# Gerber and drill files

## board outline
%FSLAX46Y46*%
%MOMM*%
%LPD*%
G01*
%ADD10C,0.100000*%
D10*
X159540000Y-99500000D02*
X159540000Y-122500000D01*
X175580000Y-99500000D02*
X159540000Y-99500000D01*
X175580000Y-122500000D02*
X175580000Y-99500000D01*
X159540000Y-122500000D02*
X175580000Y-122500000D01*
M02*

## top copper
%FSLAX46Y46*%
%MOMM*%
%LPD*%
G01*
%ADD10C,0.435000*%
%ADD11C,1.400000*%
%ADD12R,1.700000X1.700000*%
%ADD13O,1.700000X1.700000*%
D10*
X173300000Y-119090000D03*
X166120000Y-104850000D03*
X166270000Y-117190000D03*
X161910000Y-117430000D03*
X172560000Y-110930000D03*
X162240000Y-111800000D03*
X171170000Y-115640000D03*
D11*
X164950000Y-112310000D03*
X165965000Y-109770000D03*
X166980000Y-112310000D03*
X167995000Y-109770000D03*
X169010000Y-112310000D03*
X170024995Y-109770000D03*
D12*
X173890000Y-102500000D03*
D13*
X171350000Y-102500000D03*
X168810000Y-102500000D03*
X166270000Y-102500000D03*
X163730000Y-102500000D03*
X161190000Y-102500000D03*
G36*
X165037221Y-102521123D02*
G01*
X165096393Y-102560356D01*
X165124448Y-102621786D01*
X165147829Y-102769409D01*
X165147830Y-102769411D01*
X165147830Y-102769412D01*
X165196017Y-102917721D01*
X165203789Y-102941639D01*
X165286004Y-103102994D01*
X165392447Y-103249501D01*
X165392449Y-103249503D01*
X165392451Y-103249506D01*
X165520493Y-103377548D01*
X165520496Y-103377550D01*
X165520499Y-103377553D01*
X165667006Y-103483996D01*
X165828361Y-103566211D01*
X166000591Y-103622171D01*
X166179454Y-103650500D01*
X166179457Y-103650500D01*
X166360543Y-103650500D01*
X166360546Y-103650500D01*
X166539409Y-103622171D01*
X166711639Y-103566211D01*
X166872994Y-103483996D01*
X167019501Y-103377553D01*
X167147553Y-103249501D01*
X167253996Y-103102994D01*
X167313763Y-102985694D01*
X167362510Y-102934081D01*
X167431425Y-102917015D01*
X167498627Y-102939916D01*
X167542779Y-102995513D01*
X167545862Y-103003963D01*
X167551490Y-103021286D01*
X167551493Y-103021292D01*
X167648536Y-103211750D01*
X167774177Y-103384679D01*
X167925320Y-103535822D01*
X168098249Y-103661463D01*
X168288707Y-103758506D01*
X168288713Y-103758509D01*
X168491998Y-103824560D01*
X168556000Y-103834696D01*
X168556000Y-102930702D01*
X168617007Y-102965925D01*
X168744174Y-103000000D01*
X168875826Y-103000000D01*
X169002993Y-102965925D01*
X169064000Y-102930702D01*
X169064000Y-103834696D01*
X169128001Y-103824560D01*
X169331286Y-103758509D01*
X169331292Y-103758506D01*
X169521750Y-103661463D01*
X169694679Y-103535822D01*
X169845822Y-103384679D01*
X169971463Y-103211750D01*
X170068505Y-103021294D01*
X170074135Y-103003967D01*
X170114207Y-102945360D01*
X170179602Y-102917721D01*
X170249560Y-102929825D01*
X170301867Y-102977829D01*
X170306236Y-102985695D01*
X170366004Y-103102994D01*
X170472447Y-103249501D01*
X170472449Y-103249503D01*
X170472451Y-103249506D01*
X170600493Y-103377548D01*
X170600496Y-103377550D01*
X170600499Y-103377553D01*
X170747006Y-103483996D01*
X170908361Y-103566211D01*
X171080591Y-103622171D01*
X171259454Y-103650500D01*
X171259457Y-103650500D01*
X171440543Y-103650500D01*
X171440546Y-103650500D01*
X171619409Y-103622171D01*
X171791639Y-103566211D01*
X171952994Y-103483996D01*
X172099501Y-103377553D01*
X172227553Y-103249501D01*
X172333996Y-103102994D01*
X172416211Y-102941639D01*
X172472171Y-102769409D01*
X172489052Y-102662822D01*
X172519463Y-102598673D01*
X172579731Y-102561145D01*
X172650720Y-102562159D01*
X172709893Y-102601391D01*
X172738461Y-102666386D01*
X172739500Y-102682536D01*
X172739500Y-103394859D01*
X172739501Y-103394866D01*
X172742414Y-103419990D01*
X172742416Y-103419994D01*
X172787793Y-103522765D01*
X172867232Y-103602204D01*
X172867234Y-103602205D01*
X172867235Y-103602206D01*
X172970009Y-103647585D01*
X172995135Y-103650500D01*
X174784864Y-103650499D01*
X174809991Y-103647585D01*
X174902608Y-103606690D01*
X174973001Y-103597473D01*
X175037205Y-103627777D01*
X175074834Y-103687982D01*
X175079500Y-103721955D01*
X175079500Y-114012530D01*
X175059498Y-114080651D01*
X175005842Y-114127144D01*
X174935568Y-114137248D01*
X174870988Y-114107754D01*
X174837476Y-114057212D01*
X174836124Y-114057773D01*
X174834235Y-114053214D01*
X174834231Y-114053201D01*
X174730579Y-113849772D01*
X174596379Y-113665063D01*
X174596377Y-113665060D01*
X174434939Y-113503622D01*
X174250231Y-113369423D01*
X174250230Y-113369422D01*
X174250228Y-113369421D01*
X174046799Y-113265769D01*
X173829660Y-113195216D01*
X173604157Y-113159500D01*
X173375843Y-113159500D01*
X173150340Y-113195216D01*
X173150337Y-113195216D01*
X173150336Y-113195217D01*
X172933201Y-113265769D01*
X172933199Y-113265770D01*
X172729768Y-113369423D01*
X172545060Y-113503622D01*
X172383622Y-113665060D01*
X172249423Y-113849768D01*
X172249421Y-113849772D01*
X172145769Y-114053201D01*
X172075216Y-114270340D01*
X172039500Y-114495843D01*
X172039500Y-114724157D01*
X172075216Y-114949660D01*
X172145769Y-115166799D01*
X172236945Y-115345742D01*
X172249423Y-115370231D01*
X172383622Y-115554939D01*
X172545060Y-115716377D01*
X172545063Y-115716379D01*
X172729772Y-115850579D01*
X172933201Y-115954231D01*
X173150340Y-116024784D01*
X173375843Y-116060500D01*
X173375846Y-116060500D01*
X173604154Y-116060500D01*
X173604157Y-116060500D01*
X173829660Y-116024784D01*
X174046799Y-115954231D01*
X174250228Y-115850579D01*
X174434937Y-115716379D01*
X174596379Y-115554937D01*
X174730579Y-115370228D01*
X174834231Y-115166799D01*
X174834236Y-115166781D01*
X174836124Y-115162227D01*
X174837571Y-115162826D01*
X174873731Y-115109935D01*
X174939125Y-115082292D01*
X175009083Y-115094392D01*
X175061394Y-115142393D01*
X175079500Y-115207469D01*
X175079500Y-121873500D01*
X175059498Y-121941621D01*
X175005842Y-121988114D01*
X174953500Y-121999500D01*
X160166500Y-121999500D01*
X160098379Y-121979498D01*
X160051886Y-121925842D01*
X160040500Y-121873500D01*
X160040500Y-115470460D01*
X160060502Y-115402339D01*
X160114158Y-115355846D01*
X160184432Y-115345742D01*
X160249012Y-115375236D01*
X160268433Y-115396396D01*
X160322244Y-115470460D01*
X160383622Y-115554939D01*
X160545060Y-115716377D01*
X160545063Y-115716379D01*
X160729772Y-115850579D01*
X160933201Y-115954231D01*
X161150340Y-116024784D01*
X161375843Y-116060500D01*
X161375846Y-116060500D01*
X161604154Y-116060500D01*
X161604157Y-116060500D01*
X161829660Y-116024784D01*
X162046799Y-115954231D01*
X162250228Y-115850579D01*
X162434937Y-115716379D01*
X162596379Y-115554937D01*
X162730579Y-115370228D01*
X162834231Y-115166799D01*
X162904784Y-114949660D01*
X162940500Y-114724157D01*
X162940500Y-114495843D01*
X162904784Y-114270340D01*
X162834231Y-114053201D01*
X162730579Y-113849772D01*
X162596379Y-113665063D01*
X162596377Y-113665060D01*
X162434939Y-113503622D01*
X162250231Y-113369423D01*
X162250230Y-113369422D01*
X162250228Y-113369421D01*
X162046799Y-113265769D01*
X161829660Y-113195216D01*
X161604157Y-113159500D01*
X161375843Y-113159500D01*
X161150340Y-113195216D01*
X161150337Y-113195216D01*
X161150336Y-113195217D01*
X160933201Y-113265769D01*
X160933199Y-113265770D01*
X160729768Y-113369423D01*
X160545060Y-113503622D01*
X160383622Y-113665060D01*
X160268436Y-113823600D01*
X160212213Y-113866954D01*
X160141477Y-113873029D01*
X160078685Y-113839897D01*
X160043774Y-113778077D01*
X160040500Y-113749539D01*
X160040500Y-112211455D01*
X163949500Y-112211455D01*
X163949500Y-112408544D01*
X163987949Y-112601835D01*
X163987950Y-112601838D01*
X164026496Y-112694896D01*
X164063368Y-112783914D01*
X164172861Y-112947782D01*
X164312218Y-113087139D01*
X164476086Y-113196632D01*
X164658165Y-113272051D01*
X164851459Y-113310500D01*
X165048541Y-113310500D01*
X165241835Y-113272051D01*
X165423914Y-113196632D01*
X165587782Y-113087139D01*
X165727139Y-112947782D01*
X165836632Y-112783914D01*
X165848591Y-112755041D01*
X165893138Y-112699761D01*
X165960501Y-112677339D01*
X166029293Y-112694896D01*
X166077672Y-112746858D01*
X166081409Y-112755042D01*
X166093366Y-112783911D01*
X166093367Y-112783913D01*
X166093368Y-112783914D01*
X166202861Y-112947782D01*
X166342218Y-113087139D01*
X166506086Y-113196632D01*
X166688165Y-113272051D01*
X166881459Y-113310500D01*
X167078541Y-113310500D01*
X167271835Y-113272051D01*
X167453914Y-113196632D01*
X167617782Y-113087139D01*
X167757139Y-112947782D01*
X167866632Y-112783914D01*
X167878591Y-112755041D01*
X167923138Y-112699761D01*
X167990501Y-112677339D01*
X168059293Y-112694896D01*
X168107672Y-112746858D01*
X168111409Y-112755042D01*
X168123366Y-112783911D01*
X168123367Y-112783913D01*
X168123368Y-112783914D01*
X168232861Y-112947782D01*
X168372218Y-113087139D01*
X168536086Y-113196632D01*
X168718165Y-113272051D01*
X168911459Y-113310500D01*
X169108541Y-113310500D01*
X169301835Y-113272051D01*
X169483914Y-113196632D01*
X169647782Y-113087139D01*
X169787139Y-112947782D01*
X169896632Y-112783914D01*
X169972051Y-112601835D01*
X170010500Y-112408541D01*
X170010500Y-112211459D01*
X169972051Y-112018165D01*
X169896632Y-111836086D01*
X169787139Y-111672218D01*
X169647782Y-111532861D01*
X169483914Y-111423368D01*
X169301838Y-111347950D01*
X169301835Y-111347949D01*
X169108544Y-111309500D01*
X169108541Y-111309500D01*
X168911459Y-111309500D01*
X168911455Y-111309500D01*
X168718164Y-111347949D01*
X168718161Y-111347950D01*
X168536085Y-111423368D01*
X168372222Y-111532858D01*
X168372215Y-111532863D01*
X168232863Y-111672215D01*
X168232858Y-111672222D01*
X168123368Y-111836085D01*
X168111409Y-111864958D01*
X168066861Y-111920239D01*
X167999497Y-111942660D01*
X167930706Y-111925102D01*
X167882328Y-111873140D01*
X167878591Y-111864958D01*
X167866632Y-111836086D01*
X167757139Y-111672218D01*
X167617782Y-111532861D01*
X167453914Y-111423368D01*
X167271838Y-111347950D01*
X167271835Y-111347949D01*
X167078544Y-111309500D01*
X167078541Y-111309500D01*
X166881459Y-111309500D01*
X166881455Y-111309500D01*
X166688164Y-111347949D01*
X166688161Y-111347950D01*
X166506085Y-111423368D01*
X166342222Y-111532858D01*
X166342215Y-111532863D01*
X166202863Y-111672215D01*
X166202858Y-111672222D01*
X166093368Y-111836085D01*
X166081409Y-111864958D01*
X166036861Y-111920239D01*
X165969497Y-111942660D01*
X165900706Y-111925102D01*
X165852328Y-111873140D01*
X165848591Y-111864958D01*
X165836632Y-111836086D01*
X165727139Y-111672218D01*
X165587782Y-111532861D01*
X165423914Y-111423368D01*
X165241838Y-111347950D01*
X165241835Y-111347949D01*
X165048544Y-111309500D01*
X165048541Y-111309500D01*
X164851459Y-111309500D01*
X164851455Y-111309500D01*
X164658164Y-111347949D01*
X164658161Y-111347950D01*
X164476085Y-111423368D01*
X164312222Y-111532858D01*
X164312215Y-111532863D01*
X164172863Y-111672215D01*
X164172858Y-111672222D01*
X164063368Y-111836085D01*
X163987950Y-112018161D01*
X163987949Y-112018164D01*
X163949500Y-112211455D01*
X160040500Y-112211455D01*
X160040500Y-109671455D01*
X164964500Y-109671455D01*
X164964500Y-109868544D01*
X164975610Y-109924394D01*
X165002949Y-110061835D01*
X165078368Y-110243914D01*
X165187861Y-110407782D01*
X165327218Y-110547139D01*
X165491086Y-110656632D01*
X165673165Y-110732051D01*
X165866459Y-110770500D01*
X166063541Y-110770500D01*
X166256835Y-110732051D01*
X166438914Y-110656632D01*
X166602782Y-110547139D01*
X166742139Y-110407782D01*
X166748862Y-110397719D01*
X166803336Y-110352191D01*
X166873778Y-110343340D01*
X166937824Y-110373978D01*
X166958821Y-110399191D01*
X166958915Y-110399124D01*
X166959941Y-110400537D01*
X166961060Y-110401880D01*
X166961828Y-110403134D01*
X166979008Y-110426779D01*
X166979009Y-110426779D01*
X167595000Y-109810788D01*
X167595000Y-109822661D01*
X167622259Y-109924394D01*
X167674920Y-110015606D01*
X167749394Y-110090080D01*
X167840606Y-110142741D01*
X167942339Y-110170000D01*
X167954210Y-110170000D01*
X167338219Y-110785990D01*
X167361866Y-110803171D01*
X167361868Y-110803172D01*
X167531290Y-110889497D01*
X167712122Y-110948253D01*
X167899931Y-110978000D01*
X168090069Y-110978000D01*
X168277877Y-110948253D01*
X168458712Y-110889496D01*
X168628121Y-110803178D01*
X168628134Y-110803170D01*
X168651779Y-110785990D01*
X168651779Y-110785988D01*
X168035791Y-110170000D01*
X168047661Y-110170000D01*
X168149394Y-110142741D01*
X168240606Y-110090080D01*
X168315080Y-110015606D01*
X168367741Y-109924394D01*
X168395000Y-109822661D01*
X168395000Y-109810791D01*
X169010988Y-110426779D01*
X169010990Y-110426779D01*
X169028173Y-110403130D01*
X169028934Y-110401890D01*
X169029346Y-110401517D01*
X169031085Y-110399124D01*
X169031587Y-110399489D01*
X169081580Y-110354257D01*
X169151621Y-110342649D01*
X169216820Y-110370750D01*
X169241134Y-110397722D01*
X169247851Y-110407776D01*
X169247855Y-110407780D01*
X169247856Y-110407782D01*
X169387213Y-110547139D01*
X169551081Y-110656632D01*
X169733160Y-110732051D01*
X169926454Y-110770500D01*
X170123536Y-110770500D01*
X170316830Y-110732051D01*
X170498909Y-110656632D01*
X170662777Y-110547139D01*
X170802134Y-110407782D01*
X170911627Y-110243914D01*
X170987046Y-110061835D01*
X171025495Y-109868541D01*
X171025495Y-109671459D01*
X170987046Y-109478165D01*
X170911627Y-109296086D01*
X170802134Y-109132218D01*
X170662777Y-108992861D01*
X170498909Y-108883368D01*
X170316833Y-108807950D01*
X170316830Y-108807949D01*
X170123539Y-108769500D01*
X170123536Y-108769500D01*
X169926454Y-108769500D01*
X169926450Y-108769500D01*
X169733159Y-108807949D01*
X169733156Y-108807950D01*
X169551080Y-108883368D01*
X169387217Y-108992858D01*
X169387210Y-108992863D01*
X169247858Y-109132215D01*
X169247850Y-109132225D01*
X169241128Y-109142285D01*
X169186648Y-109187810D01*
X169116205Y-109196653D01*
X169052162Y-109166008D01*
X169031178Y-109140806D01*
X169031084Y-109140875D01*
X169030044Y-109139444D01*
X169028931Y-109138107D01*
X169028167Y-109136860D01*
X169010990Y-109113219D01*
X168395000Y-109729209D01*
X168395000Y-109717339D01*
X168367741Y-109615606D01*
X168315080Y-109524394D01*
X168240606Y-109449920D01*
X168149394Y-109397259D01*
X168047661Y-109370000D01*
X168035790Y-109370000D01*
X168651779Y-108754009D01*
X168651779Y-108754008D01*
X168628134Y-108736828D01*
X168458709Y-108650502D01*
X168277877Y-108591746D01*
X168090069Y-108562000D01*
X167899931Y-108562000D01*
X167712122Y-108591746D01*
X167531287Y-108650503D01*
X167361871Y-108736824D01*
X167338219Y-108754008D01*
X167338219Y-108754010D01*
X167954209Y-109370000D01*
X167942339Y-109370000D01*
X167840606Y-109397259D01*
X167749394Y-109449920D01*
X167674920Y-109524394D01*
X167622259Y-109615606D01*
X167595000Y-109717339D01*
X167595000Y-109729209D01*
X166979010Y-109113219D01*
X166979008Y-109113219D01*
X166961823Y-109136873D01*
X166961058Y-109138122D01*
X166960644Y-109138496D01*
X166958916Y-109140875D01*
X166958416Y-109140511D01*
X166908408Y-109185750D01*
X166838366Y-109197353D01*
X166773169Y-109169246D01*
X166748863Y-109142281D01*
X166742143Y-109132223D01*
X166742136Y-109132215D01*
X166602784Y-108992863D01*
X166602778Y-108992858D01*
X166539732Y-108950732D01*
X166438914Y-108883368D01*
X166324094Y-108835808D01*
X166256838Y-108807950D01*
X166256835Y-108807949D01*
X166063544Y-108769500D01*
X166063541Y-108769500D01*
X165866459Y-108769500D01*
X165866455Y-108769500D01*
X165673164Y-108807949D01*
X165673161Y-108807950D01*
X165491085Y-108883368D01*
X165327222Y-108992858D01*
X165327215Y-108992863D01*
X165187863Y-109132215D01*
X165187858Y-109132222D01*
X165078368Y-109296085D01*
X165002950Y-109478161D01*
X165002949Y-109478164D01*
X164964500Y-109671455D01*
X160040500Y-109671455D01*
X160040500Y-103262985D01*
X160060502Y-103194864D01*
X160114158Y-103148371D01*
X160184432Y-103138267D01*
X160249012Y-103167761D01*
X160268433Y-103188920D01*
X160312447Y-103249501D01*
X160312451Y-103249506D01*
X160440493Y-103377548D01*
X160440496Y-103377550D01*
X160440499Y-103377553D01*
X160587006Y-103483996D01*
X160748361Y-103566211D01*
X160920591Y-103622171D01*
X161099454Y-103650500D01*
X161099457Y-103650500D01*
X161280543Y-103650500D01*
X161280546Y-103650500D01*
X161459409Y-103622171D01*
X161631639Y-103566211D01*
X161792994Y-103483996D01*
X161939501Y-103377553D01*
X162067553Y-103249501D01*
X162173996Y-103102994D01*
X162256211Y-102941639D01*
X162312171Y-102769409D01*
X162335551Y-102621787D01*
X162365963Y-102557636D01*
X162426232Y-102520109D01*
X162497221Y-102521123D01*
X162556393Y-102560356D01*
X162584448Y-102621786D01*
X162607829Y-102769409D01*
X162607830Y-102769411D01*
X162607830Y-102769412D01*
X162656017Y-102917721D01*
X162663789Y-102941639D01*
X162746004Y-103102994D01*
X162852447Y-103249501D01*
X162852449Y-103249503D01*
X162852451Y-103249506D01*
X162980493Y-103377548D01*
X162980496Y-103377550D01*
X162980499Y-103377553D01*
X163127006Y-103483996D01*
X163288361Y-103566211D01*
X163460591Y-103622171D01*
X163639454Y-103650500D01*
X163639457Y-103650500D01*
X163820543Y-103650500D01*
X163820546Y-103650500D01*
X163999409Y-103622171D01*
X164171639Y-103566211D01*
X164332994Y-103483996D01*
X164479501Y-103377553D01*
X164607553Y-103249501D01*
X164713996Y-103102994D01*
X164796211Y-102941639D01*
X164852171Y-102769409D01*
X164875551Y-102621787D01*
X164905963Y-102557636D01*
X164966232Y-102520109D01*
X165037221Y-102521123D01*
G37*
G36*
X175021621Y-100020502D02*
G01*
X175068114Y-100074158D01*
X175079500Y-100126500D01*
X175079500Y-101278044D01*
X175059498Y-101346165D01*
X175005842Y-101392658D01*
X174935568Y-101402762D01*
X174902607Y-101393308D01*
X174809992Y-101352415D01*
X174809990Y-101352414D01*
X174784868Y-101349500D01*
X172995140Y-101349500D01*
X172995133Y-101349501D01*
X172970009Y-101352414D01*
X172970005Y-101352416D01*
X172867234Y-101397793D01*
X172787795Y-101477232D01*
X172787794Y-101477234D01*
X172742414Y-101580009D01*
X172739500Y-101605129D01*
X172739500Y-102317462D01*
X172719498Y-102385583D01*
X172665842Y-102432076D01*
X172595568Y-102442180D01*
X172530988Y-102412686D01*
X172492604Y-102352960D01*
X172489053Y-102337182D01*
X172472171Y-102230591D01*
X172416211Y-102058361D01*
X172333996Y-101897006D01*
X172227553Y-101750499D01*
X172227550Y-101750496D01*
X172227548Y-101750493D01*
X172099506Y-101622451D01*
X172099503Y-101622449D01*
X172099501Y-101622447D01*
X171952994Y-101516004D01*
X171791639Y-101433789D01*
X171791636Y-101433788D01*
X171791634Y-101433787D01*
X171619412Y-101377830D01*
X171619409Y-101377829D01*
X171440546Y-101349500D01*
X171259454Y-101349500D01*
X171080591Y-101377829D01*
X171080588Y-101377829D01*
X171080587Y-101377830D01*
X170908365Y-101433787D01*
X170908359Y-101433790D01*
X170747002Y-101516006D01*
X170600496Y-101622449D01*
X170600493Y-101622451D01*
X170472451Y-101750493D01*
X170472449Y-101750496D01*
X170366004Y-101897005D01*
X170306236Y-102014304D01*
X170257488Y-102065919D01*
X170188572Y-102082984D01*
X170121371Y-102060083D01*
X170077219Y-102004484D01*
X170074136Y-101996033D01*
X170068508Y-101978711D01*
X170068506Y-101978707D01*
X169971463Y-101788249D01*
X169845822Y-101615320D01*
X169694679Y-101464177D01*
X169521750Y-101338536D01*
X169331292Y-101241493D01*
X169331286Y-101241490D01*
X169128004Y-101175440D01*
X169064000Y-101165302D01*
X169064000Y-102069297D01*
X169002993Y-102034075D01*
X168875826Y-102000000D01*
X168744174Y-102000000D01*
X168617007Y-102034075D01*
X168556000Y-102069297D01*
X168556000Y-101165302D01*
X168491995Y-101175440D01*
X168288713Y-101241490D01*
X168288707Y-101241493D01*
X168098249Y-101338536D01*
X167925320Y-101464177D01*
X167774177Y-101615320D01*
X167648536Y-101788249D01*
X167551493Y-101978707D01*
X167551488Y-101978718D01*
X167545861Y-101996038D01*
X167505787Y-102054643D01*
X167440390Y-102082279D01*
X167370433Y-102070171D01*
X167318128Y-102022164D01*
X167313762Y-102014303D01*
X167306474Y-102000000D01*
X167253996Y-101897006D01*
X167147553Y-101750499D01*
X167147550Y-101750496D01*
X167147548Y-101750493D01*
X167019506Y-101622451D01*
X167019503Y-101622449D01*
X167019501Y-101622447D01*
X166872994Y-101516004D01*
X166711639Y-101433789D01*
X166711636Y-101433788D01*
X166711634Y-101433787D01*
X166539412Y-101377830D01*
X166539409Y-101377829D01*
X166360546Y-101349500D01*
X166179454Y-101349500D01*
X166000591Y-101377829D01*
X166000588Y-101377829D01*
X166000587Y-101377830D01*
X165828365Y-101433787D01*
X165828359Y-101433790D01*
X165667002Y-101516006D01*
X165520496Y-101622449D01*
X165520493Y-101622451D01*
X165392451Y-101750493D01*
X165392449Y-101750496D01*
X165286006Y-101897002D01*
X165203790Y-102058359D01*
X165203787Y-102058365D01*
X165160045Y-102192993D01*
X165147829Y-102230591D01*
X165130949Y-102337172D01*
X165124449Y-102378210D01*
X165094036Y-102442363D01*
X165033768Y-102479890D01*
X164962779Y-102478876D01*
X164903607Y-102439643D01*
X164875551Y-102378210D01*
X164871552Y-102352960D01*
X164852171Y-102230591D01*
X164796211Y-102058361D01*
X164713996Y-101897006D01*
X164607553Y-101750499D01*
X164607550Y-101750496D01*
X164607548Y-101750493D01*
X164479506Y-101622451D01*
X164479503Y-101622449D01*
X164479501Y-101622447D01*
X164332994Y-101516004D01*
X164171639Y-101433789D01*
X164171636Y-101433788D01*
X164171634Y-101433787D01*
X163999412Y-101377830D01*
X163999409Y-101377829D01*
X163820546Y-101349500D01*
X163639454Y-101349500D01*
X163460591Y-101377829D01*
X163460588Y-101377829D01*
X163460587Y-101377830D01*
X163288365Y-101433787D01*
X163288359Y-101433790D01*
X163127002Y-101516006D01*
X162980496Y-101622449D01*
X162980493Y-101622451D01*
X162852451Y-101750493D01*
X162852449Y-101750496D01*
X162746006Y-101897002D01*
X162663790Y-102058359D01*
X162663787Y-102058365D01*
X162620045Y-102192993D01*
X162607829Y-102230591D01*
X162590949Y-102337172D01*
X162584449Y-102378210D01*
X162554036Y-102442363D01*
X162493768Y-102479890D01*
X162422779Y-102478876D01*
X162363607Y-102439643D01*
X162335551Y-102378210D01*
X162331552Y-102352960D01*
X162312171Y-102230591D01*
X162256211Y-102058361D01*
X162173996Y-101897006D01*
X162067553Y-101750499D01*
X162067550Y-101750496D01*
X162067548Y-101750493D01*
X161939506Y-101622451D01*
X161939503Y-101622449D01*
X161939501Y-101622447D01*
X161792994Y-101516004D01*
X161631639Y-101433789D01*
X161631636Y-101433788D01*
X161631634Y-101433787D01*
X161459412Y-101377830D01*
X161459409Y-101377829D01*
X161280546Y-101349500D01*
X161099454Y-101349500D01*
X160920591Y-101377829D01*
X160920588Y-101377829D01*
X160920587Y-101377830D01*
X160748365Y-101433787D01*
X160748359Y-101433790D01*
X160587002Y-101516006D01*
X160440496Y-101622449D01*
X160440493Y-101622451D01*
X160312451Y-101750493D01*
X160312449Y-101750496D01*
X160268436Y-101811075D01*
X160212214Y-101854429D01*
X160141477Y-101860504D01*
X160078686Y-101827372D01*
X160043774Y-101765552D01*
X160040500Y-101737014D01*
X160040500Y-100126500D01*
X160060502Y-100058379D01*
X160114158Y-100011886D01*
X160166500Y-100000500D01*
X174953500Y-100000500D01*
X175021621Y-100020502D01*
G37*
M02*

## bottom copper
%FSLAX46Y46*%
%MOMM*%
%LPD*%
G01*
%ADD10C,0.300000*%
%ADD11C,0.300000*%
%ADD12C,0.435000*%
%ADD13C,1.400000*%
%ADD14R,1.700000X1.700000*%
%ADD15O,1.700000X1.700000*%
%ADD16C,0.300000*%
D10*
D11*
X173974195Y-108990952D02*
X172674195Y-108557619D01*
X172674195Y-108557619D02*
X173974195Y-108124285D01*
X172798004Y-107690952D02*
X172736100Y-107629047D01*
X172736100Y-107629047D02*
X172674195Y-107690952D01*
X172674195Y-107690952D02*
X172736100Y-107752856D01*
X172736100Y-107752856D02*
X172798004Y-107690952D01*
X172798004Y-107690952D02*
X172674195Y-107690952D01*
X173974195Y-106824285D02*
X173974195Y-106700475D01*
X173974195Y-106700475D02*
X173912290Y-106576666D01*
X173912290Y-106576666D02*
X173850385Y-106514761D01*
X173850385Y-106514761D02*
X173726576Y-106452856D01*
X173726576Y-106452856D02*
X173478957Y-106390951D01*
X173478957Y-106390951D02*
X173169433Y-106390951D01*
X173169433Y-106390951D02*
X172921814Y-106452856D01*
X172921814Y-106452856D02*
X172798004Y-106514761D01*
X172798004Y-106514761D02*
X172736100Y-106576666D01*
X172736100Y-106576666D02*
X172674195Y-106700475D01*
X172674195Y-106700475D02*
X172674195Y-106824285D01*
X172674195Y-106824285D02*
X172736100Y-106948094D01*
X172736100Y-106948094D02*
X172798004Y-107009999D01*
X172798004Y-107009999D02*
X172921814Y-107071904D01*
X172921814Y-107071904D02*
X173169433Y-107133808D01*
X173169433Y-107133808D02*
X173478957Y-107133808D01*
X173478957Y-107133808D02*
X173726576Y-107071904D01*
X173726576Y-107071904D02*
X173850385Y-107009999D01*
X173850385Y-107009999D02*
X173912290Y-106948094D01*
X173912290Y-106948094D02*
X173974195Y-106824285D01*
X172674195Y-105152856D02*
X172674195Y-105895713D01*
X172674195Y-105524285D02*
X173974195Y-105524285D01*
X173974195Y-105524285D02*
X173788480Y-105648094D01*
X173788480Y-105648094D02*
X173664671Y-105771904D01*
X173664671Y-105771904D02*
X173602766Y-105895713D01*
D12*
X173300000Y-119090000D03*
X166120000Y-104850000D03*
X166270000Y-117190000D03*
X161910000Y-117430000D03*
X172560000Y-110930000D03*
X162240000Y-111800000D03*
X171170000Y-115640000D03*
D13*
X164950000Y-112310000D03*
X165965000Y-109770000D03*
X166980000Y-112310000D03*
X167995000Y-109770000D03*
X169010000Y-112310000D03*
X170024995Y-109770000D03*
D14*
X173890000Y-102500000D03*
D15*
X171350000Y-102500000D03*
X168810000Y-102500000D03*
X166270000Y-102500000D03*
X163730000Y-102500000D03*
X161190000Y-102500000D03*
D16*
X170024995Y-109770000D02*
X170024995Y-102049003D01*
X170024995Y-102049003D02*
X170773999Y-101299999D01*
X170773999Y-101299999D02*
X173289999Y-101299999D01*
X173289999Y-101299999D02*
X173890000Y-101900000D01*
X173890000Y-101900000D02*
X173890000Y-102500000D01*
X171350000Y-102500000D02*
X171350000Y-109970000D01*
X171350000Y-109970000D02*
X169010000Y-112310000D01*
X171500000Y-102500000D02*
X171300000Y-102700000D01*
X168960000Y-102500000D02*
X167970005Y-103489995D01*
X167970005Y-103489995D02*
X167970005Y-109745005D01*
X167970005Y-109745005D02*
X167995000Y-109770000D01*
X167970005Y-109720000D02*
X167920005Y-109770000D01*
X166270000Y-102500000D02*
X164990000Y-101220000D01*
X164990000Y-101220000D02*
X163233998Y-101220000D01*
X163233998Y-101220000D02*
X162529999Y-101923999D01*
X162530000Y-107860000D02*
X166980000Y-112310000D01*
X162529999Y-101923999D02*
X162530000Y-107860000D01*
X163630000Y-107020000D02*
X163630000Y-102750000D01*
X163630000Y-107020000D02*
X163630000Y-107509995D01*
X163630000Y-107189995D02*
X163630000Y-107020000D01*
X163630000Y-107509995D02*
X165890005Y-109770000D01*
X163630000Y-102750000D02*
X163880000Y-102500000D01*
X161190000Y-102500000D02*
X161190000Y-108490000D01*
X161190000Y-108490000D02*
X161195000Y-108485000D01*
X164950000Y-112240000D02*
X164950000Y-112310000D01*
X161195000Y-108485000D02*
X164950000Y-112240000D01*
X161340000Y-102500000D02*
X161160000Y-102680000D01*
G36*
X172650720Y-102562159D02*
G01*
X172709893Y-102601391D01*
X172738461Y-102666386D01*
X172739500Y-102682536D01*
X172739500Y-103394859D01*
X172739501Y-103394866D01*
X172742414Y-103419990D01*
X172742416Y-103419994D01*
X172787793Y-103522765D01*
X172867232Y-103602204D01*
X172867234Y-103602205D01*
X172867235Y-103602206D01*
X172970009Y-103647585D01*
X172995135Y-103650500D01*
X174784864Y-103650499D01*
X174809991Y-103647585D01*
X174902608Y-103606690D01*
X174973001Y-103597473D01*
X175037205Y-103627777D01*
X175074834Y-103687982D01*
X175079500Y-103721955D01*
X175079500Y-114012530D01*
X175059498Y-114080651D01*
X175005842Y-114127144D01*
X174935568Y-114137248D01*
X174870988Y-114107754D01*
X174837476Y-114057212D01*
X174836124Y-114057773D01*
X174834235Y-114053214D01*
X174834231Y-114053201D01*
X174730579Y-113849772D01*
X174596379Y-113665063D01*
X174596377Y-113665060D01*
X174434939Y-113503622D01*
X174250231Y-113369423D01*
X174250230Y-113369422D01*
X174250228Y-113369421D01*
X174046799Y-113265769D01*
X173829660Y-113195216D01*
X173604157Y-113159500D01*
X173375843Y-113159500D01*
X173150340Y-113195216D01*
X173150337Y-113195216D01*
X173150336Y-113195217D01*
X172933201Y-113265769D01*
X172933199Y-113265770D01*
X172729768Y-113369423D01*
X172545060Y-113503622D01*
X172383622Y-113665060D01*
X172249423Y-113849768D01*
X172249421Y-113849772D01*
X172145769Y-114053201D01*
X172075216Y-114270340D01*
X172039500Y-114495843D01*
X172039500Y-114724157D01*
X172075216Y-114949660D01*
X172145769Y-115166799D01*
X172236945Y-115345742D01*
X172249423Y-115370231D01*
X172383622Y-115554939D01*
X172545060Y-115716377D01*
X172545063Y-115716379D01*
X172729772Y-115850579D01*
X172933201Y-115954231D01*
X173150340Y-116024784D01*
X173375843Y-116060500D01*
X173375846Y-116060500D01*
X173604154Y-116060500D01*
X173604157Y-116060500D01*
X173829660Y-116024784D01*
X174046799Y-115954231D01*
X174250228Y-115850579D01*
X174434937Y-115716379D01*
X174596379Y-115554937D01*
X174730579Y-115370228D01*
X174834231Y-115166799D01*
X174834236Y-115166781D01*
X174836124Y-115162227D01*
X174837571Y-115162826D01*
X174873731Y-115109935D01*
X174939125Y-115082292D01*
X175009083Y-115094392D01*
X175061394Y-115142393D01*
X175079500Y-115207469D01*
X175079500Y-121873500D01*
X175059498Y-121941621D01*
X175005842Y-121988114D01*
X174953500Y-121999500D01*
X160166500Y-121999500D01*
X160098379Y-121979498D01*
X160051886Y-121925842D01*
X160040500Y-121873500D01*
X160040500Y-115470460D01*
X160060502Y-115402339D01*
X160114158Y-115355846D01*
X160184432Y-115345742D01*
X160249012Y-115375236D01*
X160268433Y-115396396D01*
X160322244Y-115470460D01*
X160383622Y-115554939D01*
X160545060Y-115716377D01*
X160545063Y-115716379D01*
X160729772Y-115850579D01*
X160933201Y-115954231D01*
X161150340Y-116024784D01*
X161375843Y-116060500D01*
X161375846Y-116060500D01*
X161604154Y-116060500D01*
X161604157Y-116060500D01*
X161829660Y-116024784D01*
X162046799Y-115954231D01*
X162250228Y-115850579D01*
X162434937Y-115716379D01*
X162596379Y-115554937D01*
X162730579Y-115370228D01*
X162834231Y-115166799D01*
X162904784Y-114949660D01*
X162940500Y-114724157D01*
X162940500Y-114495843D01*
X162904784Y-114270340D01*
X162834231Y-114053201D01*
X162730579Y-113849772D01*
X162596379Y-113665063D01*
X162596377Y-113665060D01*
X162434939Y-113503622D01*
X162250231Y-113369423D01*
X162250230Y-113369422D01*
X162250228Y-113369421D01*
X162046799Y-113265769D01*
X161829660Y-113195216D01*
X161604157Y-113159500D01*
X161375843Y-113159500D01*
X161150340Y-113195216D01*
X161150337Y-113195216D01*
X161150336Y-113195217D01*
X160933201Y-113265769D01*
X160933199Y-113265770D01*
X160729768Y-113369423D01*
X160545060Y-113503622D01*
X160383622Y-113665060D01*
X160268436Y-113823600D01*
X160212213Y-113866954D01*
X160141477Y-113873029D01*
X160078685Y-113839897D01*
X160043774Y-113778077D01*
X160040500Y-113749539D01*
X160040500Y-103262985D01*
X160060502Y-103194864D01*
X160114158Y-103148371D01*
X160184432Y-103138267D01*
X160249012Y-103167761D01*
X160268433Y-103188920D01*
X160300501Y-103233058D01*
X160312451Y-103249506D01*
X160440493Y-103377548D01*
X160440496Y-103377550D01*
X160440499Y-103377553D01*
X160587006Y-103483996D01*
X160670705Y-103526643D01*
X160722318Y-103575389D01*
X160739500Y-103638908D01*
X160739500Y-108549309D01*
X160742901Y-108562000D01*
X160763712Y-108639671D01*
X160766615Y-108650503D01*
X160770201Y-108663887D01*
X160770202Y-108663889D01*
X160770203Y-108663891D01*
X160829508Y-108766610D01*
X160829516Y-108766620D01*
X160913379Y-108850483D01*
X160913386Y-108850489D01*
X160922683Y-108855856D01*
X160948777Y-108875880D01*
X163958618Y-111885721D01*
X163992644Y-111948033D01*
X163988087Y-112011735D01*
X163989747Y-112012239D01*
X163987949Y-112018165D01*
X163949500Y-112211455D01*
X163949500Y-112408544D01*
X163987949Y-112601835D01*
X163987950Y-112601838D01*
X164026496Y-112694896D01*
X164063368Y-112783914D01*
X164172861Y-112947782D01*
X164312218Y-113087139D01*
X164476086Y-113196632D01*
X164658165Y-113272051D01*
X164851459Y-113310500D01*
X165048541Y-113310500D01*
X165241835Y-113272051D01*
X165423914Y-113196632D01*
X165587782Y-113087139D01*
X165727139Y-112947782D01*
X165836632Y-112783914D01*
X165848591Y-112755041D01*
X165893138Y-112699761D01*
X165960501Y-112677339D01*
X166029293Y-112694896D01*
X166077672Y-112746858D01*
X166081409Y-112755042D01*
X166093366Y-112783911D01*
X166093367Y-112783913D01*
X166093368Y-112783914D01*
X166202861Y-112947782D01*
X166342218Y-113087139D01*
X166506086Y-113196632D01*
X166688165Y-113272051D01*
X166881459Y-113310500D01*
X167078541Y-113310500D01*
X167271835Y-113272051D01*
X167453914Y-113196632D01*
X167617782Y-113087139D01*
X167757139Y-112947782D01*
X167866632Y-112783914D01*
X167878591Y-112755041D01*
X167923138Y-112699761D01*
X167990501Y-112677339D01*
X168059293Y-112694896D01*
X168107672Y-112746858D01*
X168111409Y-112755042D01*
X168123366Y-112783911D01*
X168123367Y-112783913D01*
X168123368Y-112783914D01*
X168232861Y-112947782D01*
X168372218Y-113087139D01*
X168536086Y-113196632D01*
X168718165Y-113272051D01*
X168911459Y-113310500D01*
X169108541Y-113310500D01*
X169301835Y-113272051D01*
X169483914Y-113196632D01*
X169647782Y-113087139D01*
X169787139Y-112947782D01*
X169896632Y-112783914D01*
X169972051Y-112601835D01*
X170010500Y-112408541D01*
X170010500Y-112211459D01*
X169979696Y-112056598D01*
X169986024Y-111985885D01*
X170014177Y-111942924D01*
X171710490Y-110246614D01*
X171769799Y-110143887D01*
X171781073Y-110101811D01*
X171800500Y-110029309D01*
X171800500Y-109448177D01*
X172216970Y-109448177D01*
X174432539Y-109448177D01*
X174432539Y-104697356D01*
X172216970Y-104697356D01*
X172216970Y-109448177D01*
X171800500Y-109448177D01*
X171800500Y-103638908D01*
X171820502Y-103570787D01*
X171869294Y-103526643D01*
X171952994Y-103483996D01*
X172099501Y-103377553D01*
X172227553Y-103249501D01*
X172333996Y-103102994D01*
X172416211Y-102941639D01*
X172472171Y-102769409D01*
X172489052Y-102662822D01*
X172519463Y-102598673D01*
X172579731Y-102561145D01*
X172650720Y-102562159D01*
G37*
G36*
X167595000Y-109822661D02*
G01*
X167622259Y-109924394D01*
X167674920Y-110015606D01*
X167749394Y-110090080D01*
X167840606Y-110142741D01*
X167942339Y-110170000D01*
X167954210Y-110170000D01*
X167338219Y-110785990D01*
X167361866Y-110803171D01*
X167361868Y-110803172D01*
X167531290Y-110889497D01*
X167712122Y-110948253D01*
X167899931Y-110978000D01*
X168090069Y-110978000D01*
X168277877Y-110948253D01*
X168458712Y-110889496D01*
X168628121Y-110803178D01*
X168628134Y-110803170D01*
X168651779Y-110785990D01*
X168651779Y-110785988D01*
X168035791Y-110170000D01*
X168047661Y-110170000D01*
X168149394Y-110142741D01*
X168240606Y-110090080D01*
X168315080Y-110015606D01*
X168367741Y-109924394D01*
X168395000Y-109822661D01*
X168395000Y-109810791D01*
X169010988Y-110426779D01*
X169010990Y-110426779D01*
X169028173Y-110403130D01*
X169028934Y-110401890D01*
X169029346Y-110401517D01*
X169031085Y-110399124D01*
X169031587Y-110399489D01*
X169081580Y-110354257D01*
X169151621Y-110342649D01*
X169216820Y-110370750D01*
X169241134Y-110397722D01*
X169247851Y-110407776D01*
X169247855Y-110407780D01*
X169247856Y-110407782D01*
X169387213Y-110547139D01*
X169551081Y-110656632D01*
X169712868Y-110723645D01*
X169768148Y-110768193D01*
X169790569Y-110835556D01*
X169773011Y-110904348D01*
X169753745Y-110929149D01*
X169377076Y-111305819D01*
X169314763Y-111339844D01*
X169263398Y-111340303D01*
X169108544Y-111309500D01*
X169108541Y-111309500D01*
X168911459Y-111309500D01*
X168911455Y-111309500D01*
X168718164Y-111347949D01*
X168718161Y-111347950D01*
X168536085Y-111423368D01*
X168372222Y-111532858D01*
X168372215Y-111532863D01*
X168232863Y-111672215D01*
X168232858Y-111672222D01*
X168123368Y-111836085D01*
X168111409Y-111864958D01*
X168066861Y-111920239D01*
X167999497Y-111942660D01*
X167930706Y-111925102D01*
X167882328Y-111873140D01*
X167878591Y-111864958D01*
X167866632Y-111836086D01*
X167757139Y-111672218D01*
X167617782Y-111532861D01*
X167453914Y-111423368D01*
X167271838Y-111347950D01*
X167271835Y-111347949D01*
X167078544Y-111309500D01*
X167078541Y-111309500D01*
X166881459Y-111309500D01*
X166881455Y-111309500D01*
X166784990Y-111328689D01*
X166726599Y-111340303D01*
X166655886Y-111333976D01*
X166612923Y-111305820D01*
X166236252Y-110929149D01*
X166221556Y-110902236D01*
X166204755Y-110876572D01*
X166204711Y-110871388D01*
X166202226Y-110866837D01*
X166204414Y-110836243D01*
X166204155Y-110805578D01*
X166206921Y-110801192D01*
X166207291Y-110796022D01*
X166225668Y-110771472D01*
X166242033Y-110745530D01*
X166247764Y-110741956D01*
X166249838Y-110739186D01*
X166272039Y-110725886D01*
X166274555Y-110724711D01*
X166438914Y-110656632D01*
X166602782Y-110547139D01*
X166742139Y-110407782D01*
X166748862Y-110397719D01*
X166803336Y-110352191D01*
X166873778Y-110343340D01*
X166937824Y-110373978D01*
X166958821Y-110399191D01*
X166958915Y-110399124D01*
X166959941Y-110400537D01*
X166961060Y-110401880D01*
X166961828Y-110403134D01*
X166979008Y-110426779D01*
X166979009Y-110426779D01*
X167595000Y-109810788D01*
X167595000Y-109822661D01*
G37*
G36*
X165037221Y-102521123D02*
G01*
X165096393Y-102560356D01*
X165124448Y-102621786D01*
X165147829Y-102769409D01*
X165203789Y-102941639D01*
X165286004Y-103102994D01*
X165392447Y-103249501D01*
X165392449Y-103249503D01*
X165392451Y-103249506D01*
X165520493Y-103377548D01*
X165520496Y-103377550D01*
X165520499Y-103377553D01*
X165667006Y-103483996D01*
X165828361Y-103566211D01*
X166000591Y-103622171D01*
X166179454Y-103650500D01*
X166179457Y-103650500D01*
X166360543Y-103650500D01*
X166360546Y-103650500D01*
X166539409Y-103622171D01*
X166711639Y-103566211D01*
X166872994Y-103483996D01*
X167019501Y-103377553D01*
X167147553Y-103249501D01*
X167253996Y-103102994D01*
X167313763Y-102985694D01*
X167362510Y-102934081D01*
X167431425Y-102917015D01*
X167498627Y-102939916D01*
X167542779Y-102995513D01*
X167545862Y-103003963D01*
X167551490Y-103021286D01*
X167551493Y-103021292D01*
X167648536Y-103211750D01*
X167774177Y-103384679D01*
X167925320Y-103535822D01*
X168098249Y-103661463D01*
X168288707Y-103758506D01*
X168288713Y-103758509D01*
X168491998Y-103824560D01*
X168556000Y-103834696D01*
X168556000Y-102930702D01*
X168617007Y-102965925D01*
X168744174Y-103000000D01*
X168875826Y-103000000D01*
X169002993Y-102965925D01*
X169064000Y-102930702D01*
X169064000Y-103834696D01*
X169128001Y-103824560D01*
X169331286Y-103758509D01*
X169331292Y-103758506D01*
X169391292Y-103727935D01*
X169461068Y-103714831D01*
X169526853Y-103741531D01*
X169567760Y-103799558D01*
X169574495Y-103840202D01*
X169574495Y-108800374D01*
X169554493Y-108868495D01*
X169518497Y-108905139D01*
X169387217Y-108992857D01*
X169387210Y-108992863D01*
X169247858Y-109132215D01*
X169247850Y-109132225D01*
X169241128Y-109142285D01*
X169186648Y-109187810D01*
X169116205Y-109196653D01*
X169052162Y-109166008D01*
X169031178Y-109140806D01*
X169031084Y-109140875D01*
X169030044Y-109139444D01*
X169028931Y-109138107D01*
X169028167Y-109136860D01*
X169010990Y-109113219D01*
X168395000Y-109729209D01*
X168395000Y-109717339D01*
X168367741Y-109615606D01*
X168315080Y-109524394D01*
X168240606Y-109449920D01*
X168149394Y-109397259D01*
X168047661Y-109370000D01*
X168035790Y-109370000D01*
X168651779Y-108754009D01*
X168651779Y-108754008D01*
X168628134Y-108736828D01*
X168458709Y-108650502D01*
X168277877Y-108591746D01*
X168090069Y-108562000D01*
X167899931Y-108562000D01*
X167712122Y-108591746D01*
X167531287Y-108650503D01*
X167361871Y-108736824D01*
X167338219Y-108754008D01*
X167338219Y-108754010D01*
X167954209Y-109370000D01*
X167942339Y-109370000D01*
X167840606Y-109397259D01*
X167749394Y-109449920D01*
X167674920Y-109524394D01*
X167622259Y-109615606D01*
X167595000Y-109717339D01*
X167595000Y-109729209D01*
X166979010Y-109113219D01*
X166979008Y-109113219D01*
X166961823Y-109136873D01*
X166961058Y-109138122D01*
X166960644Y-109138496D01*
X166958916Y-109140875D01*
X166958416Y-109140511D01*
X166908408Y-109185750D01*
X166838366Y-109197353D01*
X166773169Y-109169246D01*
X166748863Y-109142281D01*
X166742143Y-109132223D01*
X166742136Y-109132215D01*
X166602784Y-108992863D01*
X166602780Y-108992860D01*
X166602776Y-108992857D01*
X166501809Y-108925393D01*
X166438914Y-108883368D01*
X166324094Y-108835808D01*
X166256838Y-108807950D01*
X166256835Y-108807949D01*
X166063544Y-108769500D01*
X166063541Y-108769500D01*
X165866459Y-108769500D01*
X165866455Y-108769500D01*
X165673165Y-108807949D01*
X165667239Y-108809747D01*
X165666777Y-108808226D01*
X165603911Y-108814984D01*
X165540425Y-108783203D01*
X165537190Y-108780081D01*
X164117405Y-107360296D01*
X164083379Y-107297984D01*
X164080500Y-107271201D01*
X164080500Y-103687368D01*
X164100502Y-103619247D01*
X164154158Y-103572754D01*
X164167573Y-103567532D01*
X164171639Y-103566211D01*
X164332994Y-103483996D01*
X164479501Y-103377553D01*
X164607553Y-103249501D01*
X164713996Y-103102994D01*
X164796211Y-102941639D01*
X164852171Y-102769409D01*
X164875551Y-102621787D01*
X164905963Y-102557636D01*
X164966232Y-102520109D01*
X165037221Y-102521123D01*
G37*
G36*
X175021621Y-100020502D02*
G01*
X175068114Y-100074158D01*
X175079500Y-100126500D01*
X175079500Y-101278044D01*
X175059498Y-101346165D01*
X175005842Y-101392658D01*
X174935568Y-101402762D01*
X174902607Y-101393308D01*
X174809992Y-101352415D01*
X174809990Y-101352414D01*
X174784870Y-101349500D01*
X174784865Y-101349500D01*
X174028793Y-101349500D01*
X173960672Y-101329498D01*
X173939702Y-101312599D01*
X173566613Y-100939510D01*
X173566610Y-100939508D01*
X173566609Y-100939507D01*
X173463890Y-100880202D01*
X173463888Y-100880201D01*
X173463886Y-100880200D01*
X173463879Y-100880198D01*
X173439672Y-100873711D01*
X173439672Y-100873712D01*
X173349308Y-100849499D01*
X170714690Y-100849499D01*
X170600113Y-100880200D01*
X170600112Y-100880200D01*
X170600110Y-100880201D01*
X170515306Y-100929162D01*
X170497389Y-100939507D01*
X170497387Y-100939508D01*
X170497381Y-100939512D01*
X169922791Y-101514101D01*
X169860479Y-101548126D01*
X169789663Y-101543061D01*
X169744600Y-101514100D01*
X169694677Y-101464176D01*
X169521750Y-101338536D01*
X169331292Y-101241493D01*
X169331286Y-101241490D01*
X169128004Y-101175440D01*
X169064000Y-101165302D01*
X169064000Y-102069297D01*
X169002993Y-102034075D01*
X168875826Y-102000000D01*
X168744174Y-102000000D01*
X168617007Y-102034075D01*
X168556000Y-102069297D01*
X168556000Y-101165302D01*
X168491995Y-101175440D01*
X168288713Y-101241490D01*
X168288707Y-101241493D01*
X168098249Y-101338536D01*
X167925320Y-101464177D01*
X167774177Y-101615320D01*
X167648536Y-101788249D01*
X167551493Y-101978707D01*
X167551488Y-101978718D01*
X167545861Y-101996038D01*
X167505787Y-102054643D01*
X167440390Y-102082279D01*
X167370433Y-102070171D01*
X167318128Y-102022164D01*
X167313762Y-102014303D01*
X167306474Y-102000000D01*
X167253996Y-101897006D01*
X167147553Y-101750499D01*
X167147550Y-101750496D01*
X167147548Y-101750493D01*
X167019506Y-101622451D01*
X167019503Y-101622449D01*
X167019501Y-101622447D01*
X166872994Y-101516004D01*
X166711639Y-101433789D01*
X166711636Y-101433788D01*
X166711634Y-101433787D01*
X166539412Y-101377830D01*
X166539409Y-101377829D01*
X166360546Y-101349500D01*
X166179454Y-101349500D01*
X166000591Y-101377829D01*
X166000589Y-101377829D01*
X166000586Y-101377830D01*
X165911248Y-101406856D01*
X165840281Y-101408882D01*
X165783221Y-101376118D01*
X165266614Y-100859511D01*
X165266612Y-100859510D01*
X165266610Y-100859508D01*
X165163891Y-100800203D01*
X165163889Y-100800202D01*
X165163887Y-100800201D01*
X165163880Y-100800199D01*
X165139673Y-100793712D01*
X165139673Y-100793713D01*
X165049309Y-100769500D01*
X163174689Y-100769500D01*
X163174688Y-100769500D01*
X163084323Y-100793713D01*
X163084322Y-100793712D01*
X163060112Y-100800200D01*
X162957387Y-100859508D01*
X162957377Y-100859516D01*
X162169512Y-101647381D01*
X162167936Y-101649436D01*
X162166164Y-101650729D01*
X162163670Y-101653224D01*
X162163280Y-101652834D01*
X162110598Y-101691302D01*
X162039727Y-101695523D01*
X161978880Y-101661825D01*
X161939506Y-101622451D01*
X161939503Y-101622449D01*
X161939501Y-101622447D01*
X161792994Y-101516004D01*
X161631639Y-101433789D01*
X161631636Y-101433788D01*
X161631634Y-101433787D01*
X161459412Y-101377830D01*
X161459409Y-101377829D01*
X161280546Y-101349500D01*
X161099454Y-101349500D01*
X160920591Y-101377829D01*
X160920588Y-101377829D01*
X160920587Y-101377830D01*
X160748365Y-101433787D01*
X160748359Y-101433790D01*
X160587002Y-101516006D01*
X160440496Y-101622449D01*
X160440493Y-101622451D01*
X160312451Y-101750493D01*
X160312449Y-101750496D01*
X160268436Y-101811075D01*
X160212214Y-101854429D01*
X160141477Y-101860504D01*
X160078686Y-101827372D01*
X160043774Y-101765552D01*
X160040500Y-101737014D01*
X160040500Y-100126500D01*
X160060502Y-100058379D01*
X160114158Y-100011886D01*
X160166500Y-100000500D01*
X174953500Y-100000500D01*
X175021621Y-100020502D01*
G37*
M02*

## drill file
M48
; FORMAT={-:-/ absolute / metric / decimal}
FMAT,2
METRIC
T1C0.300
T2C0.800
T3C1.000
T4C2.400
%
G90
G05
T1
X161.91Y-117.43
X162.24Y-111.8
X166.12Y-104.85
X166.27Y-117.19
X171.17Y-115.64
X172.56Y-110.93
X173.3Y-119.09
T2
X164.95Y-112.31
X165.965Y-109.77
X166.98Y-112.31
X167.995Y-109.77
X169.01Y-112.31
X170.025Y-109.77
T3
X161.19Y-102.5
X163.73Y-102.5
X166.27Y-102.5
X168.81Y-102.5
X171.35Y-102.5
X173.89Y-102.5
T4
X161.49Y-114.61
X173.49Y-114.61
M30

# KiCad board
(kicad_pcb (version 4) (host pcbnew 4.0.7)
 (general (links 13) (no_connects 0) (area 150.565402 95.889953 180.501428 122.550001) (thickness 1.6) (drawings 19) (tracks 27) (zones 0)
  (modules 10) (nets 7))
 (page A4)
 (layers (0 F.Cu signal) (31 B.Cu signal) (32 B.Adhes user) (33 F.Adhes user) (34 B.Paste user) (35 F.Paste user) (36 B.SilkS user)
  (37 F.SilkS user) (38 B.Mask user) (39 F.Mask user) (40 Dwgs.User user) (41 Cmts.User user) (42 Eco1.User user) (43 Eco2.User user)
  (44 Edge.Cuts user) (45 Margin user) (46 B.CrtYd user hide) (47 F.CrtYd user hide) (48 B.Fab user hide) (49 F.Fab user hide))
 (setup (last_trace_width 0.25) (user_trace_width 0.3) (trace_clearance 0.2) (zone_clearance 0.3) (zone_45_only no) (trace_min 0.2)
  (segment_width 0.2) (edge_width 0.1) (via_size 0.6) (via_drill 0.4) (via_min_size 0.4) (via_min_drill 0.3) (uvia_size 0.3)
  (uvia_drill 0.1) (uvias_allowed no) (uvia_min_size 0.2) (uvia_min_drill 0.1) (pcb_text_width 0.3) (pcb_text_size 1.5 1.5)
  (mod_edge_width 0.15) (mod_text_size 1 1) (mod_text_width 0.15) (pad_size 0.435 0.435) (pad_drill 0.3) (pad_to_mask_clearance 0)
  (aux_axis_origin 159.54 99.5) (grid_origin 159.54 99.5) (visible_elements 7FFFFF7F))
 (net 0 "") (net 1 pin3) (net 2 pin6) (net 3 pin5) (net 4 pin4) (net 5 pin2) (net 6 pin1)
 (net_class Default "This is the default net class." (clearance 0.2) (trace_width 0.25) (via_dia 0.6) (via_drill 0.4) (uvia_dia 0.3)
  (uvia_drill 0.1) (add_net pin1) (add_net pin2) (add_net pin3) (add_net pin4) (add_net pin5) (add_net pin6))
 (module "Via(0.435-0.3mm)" (layer F.Cu) (at 173.3 119.09)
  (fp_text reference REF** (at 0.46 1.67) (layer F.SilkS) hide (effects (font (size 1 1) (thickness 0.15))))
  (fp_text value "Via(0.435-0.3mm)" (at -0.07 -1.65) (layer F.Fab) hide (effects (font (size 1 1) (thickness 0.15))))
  (pad 1 thru_hole circle (at 0 0) (size 0.435 0.435) (drill 0.3) (layers *.Cu) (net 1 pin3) (zone_connect 2)))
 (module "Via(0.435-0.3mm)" (layer F.Cu) (at 166.12 104.85)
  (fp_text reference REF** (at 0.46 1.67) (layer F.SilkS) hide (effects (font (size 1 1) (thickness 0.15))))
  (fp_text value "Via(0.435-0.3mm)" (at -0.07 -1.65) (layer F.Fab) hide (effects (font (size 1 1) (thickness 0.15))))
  (pad 1 thru_hole circle (at 0 0) (size 0.435 0.435) (drill 0.3) (layers *.Cu) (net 1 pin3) (zone_connect 2)))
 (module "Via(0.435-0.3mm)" (layer F.Cu) (at 166.27 117.19)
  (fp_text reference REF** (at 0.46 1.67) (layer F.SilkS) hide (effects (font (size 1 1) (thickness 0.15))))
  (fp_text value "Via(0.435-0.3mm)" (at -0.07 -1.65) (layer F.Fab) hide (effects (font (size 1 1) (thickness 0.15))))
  (pad 1 thru_hole circle (at 0 0) (size 0.435 0.435) (drill 0.3) (layers *.Cu) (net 1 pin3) (zone_connect 2)))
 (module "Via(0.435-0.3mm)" (layer F.Cu) (at 161.91 117.43)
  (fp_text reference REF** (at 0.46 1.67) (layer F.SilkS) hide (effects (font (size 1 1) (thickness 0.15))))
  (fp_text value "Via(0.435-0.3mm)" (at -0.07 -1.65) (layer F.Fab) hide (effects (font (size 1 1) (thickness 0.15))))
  (pad 1 thru_hole circle (at 0 0) (size 0.435 0.435) (drill 0.3) (layers *.Cu) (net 1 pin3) (zone_connect 2)))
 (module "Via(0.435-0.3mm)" (layer F.Cu) (at 172.56 110.93)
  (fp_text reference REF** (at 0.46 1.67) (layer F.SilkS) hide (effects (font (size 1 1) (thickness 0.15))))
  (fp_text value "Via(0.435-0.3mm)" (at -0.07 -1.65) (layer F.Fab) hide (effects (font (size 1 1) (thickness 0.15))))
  (pad 1 thru_hole circle (at 0 0) (size 0.435 0.435) (drill 0.3) (layers *.Cu) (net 1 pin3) (zone_connect 2)))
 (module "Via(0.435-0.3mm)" (layer F.Cu) (at 162.24 111.8)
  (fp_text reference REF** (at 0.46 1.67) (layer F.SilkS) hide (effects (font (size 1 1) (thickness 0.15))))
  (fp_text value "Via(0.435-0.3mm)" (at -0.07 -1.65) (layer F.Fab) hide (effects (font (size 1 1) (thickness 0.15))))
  (pad 1 thru_hole circle (at 0 0) (size 0.435 0.435) (drill 0.3) (layers *.Cu) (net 1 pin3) (zone_connect 2)))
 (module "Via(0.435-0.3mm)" (layer F.Cu) (at 171.17 115.64)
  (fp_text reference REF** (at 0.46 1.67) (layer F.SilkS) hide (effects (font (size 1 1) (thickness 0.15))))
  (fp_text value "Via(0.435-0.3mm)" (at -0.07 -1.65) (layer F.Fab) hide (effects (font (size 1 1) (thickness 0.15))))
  (pad 1 thru_hole circle (at 0 0) (size 0.435 0.435) (drill 0.3) (layers *.Cu) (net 1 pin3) (zone_connect 2)))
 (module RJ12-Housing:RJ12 (layer F.Cu) (at 165.19 113.42)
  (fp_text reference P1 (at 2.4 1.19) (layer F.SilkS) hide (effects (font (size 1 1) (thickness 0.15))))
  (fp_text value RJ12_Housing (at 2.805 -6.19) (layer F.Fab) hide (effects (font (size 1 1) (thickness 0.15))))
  (pad "" np_thru_hole circle (at -3.7 1.19) (size 2.4 2.4) (drill 2.4) (layers *.Cu *.Mask))
  (pad "" np_thru_hole circle (at 8.3 1.19) (size 2.4 2.4) (drill 2.4) (layers *.Cu *.Mask))
  (pad 6 thru_hole circle (at -0.24 -1.11) (size 1.4 1.4) (drill 0.8) (layers *.Cu *.Mask) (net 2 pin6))
  (pad 5 thru_hole circle (at 0.775 -3.65) (size 1.4 1.4) (drill 0.8) (layers *.Cu *.Mask) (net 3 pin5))
  (pad 4 thru_hole circle (at 1.79 -1.11) (size 1.4 1.4) (drill 0.8) (layers *.Cu *.Mask) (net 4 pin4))
  (pad 3 thru_hole circle (at 2.805 -3.65) (size 1.4 1.4) (drill 0.8) (layers *.Cu *.Mask) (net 1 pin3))
  (pad 2 thru_hole circle (at 3.82 -1.11) (size 1.4 1.4) (drill 0.8) (layers *.Cu *.Mask) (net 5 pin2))
  (pad 1 thru_hole circle (at 4.834995 -3.65) (size 1.4 1.4) (drill 0.8) (layers *.Cu *.Mask) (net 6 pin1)))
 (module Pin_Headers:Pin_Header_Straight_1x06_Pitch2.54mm (layer B.Cu) (at 173.89 102.5 90)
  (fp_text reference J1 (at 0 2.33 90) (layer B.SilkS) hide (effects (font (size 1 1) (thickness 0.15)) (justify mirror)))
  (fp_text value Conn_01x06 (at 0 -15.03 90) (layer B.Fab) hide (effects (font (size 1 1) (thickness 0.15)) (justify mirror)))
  (pad 1 thru_hole rect (at 0 0 90) (size 1.7 1.7) (drill 1) (layers *.Cu *.Mask) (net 6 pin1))
  (pad 2 thru_hole oval (at 0 -2.54 90) (size 1.7 1.7) (drill 1) (layers *.Cu *.Mask) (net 5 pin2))
  (pad 3 thru_hole oval (at 0 -5.08 90) (size 1.7 1.7) (drill 1) (layers *.Cu *.Mask) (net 1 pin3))
  (pad 4 thru_hole oval (at 0 -7.62 90) (size 1.7 1.7) (drill 1) (layers *.Cu *.Mask) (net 4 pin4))
  (pad 5 thru_hole oval (at 0 -10.16 90) (size 1.7 1.7) (drill 1) (layers *.Cu *.Mask) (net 3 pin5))
  (pad 6 thru_hole oval (at 0 -12.7 90) (size 1.7 1.7) (drill 1) (layers *.Cu *.Mask) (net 2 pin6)))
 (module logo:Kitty (layer B.Cu) (at 167.84 115.91 180)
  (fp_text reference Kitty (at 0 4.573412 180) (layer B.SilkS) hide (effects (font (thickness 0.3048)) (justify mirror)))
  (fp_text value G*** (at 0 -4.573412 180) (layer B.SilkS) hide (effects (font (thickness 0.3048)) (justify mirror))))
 (gr_line (start 159.54 99.5) (end 159.54 122.5) (layer Edge.Cuts) (width 0.1))
 (gr_line (start 175.58 99.5) (end 159.54 99.5) (layer Edge.Cuts) (width 0.1))
 (gr_line (start 175.58 122.5) (end 175.58 99.5) (layer Edge.Cuts) (width 0.1))
 (gr_line (start 159.54 122.5) (end 175.58 122.5) (layer Edge.Cuts) (width 0.1))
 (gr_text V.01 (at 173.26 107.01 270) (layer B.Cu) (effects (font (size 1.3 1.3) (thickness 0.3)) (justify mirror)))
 (segment (start 170.024995 109.77) (end 170.024995 102.049003) (width 0.3) (layer B.Cu) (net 6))
 (segment (start 170.024995 102.049003) (end 170.773999 101.299999) (width 0.3) (layer B.Cu) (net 6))
 (segment (start 170.773999 101.299999) (end 173.289999 101.299999) (width 0.3) (layer B.Cu) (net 6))
 (segment (start 173.289999 101.299999) (end 173.89 101.9) (width 0.3) (layer B.Cu) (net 6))
 (segment (start 173.89 101.9) (end 173.89 102.5) (width 0.3) (layer B.Cu) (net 6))
 (segment (start 171.35 102.5) (end 171.35 109.97) (width 0.3) (layer B.Cu) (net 5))
 (segment (start 171.35 109.97) (end 169.01 112.31) (width 0.3) (layer B.Cu) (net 5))
 (segment (start 171.5 102.5) (end 171.3 102.7) (width 0.3) (layer B.Cu) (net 5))
 (segment (start 168.96 102.5) (end 167.970005 103.489995) (width 0.3) (layer B.Cu) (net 1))
 (segment (start 167.970005 103.489995) (end 167.970005 109.745005) (width 0.3) (layer B.Cu) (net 1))
 (segment (start 167.970005 109.745005) (end 167.995 109.77) (width 0.3) (layer B.Cu) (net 1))
 (segment (start 167.970005 109.72) (end 167.920005 109.77) (width 0.3) (layer B.Cu) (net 1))
 (segment (start 166.27 102.5) (end 164.99 101.22) (width 0.3) (layer B.Cu) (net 4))
 (segment (start 164.99 101.22) (end 163.233998 101.22) (width 0.3) (layer B.Cu) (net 4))
 (segment (start 163.233998 101.22) (end 162.529999 101.923999) (width 0.3) (layer B.Cu) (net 4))
 (segment (start 162.53 107.86) (end 166.98 112.31) (width 0.3) (layer B.Cu) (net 4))
 (segment (start 162.529999 101.923999) (end 162.53 107.86) (width 0.3) (layer B.Cu) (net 4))
 (segment (start 163.63 107.02) (end 163.63 102.75) (width 0.3) (layer B.Cu) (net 3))
 (segment (start 163.63 107.02) (end 163.63 107.509995) (width 0.3) (layer B.Cu) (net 3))
 (segment (start 163.63 107.189995) (end 163.63 107.02) (width 0.3) (layer B.Cu) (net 3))
 (segment (start 163.63 107.509995) (end 165.890005 109.77) (width 0.3) (layer B.Cu) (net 3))
 (segment (start 163.63 102.75) (end 163.88 102.5) (width 0.3) (layer B.Cu) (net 3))
 (segment (start 161.19 102.5) (end 161.19 108.49) (width 0.3) (layer B.Cu) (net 2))
 (segment (start 161.19 108.49) (end 161.195 108.485) (width 0.3) (layer B.Cu) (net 2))
 (segment (start 164.95 112.24) (end 164.95 112.31) (width 0.3) (layer B.Cu) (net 2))
 (segment (start 161.195 108.485) (end 164.95 112.24) (width 0.3) (layer B.Cu) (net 2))
 (segment (start 161.34 102.5) (end 161.16 102.68) (width 0.3) (layer B.Cu) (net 2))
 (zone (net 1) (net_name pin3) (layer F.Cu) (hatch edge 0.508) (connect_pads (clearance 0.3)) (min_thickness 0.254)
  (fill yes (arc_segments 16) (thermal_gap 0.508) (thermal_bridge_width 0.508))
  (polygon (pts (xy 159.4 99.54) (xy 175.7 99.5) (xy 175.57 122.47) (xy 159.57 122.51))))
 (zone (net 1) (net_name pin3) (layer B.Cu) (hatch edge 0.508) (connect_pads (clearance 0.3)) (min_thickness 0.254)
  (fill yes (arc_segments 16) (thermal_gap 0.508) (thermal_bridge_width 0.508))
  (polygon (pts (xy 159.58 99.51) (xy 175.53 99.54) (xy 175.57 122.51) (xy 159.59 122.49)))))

